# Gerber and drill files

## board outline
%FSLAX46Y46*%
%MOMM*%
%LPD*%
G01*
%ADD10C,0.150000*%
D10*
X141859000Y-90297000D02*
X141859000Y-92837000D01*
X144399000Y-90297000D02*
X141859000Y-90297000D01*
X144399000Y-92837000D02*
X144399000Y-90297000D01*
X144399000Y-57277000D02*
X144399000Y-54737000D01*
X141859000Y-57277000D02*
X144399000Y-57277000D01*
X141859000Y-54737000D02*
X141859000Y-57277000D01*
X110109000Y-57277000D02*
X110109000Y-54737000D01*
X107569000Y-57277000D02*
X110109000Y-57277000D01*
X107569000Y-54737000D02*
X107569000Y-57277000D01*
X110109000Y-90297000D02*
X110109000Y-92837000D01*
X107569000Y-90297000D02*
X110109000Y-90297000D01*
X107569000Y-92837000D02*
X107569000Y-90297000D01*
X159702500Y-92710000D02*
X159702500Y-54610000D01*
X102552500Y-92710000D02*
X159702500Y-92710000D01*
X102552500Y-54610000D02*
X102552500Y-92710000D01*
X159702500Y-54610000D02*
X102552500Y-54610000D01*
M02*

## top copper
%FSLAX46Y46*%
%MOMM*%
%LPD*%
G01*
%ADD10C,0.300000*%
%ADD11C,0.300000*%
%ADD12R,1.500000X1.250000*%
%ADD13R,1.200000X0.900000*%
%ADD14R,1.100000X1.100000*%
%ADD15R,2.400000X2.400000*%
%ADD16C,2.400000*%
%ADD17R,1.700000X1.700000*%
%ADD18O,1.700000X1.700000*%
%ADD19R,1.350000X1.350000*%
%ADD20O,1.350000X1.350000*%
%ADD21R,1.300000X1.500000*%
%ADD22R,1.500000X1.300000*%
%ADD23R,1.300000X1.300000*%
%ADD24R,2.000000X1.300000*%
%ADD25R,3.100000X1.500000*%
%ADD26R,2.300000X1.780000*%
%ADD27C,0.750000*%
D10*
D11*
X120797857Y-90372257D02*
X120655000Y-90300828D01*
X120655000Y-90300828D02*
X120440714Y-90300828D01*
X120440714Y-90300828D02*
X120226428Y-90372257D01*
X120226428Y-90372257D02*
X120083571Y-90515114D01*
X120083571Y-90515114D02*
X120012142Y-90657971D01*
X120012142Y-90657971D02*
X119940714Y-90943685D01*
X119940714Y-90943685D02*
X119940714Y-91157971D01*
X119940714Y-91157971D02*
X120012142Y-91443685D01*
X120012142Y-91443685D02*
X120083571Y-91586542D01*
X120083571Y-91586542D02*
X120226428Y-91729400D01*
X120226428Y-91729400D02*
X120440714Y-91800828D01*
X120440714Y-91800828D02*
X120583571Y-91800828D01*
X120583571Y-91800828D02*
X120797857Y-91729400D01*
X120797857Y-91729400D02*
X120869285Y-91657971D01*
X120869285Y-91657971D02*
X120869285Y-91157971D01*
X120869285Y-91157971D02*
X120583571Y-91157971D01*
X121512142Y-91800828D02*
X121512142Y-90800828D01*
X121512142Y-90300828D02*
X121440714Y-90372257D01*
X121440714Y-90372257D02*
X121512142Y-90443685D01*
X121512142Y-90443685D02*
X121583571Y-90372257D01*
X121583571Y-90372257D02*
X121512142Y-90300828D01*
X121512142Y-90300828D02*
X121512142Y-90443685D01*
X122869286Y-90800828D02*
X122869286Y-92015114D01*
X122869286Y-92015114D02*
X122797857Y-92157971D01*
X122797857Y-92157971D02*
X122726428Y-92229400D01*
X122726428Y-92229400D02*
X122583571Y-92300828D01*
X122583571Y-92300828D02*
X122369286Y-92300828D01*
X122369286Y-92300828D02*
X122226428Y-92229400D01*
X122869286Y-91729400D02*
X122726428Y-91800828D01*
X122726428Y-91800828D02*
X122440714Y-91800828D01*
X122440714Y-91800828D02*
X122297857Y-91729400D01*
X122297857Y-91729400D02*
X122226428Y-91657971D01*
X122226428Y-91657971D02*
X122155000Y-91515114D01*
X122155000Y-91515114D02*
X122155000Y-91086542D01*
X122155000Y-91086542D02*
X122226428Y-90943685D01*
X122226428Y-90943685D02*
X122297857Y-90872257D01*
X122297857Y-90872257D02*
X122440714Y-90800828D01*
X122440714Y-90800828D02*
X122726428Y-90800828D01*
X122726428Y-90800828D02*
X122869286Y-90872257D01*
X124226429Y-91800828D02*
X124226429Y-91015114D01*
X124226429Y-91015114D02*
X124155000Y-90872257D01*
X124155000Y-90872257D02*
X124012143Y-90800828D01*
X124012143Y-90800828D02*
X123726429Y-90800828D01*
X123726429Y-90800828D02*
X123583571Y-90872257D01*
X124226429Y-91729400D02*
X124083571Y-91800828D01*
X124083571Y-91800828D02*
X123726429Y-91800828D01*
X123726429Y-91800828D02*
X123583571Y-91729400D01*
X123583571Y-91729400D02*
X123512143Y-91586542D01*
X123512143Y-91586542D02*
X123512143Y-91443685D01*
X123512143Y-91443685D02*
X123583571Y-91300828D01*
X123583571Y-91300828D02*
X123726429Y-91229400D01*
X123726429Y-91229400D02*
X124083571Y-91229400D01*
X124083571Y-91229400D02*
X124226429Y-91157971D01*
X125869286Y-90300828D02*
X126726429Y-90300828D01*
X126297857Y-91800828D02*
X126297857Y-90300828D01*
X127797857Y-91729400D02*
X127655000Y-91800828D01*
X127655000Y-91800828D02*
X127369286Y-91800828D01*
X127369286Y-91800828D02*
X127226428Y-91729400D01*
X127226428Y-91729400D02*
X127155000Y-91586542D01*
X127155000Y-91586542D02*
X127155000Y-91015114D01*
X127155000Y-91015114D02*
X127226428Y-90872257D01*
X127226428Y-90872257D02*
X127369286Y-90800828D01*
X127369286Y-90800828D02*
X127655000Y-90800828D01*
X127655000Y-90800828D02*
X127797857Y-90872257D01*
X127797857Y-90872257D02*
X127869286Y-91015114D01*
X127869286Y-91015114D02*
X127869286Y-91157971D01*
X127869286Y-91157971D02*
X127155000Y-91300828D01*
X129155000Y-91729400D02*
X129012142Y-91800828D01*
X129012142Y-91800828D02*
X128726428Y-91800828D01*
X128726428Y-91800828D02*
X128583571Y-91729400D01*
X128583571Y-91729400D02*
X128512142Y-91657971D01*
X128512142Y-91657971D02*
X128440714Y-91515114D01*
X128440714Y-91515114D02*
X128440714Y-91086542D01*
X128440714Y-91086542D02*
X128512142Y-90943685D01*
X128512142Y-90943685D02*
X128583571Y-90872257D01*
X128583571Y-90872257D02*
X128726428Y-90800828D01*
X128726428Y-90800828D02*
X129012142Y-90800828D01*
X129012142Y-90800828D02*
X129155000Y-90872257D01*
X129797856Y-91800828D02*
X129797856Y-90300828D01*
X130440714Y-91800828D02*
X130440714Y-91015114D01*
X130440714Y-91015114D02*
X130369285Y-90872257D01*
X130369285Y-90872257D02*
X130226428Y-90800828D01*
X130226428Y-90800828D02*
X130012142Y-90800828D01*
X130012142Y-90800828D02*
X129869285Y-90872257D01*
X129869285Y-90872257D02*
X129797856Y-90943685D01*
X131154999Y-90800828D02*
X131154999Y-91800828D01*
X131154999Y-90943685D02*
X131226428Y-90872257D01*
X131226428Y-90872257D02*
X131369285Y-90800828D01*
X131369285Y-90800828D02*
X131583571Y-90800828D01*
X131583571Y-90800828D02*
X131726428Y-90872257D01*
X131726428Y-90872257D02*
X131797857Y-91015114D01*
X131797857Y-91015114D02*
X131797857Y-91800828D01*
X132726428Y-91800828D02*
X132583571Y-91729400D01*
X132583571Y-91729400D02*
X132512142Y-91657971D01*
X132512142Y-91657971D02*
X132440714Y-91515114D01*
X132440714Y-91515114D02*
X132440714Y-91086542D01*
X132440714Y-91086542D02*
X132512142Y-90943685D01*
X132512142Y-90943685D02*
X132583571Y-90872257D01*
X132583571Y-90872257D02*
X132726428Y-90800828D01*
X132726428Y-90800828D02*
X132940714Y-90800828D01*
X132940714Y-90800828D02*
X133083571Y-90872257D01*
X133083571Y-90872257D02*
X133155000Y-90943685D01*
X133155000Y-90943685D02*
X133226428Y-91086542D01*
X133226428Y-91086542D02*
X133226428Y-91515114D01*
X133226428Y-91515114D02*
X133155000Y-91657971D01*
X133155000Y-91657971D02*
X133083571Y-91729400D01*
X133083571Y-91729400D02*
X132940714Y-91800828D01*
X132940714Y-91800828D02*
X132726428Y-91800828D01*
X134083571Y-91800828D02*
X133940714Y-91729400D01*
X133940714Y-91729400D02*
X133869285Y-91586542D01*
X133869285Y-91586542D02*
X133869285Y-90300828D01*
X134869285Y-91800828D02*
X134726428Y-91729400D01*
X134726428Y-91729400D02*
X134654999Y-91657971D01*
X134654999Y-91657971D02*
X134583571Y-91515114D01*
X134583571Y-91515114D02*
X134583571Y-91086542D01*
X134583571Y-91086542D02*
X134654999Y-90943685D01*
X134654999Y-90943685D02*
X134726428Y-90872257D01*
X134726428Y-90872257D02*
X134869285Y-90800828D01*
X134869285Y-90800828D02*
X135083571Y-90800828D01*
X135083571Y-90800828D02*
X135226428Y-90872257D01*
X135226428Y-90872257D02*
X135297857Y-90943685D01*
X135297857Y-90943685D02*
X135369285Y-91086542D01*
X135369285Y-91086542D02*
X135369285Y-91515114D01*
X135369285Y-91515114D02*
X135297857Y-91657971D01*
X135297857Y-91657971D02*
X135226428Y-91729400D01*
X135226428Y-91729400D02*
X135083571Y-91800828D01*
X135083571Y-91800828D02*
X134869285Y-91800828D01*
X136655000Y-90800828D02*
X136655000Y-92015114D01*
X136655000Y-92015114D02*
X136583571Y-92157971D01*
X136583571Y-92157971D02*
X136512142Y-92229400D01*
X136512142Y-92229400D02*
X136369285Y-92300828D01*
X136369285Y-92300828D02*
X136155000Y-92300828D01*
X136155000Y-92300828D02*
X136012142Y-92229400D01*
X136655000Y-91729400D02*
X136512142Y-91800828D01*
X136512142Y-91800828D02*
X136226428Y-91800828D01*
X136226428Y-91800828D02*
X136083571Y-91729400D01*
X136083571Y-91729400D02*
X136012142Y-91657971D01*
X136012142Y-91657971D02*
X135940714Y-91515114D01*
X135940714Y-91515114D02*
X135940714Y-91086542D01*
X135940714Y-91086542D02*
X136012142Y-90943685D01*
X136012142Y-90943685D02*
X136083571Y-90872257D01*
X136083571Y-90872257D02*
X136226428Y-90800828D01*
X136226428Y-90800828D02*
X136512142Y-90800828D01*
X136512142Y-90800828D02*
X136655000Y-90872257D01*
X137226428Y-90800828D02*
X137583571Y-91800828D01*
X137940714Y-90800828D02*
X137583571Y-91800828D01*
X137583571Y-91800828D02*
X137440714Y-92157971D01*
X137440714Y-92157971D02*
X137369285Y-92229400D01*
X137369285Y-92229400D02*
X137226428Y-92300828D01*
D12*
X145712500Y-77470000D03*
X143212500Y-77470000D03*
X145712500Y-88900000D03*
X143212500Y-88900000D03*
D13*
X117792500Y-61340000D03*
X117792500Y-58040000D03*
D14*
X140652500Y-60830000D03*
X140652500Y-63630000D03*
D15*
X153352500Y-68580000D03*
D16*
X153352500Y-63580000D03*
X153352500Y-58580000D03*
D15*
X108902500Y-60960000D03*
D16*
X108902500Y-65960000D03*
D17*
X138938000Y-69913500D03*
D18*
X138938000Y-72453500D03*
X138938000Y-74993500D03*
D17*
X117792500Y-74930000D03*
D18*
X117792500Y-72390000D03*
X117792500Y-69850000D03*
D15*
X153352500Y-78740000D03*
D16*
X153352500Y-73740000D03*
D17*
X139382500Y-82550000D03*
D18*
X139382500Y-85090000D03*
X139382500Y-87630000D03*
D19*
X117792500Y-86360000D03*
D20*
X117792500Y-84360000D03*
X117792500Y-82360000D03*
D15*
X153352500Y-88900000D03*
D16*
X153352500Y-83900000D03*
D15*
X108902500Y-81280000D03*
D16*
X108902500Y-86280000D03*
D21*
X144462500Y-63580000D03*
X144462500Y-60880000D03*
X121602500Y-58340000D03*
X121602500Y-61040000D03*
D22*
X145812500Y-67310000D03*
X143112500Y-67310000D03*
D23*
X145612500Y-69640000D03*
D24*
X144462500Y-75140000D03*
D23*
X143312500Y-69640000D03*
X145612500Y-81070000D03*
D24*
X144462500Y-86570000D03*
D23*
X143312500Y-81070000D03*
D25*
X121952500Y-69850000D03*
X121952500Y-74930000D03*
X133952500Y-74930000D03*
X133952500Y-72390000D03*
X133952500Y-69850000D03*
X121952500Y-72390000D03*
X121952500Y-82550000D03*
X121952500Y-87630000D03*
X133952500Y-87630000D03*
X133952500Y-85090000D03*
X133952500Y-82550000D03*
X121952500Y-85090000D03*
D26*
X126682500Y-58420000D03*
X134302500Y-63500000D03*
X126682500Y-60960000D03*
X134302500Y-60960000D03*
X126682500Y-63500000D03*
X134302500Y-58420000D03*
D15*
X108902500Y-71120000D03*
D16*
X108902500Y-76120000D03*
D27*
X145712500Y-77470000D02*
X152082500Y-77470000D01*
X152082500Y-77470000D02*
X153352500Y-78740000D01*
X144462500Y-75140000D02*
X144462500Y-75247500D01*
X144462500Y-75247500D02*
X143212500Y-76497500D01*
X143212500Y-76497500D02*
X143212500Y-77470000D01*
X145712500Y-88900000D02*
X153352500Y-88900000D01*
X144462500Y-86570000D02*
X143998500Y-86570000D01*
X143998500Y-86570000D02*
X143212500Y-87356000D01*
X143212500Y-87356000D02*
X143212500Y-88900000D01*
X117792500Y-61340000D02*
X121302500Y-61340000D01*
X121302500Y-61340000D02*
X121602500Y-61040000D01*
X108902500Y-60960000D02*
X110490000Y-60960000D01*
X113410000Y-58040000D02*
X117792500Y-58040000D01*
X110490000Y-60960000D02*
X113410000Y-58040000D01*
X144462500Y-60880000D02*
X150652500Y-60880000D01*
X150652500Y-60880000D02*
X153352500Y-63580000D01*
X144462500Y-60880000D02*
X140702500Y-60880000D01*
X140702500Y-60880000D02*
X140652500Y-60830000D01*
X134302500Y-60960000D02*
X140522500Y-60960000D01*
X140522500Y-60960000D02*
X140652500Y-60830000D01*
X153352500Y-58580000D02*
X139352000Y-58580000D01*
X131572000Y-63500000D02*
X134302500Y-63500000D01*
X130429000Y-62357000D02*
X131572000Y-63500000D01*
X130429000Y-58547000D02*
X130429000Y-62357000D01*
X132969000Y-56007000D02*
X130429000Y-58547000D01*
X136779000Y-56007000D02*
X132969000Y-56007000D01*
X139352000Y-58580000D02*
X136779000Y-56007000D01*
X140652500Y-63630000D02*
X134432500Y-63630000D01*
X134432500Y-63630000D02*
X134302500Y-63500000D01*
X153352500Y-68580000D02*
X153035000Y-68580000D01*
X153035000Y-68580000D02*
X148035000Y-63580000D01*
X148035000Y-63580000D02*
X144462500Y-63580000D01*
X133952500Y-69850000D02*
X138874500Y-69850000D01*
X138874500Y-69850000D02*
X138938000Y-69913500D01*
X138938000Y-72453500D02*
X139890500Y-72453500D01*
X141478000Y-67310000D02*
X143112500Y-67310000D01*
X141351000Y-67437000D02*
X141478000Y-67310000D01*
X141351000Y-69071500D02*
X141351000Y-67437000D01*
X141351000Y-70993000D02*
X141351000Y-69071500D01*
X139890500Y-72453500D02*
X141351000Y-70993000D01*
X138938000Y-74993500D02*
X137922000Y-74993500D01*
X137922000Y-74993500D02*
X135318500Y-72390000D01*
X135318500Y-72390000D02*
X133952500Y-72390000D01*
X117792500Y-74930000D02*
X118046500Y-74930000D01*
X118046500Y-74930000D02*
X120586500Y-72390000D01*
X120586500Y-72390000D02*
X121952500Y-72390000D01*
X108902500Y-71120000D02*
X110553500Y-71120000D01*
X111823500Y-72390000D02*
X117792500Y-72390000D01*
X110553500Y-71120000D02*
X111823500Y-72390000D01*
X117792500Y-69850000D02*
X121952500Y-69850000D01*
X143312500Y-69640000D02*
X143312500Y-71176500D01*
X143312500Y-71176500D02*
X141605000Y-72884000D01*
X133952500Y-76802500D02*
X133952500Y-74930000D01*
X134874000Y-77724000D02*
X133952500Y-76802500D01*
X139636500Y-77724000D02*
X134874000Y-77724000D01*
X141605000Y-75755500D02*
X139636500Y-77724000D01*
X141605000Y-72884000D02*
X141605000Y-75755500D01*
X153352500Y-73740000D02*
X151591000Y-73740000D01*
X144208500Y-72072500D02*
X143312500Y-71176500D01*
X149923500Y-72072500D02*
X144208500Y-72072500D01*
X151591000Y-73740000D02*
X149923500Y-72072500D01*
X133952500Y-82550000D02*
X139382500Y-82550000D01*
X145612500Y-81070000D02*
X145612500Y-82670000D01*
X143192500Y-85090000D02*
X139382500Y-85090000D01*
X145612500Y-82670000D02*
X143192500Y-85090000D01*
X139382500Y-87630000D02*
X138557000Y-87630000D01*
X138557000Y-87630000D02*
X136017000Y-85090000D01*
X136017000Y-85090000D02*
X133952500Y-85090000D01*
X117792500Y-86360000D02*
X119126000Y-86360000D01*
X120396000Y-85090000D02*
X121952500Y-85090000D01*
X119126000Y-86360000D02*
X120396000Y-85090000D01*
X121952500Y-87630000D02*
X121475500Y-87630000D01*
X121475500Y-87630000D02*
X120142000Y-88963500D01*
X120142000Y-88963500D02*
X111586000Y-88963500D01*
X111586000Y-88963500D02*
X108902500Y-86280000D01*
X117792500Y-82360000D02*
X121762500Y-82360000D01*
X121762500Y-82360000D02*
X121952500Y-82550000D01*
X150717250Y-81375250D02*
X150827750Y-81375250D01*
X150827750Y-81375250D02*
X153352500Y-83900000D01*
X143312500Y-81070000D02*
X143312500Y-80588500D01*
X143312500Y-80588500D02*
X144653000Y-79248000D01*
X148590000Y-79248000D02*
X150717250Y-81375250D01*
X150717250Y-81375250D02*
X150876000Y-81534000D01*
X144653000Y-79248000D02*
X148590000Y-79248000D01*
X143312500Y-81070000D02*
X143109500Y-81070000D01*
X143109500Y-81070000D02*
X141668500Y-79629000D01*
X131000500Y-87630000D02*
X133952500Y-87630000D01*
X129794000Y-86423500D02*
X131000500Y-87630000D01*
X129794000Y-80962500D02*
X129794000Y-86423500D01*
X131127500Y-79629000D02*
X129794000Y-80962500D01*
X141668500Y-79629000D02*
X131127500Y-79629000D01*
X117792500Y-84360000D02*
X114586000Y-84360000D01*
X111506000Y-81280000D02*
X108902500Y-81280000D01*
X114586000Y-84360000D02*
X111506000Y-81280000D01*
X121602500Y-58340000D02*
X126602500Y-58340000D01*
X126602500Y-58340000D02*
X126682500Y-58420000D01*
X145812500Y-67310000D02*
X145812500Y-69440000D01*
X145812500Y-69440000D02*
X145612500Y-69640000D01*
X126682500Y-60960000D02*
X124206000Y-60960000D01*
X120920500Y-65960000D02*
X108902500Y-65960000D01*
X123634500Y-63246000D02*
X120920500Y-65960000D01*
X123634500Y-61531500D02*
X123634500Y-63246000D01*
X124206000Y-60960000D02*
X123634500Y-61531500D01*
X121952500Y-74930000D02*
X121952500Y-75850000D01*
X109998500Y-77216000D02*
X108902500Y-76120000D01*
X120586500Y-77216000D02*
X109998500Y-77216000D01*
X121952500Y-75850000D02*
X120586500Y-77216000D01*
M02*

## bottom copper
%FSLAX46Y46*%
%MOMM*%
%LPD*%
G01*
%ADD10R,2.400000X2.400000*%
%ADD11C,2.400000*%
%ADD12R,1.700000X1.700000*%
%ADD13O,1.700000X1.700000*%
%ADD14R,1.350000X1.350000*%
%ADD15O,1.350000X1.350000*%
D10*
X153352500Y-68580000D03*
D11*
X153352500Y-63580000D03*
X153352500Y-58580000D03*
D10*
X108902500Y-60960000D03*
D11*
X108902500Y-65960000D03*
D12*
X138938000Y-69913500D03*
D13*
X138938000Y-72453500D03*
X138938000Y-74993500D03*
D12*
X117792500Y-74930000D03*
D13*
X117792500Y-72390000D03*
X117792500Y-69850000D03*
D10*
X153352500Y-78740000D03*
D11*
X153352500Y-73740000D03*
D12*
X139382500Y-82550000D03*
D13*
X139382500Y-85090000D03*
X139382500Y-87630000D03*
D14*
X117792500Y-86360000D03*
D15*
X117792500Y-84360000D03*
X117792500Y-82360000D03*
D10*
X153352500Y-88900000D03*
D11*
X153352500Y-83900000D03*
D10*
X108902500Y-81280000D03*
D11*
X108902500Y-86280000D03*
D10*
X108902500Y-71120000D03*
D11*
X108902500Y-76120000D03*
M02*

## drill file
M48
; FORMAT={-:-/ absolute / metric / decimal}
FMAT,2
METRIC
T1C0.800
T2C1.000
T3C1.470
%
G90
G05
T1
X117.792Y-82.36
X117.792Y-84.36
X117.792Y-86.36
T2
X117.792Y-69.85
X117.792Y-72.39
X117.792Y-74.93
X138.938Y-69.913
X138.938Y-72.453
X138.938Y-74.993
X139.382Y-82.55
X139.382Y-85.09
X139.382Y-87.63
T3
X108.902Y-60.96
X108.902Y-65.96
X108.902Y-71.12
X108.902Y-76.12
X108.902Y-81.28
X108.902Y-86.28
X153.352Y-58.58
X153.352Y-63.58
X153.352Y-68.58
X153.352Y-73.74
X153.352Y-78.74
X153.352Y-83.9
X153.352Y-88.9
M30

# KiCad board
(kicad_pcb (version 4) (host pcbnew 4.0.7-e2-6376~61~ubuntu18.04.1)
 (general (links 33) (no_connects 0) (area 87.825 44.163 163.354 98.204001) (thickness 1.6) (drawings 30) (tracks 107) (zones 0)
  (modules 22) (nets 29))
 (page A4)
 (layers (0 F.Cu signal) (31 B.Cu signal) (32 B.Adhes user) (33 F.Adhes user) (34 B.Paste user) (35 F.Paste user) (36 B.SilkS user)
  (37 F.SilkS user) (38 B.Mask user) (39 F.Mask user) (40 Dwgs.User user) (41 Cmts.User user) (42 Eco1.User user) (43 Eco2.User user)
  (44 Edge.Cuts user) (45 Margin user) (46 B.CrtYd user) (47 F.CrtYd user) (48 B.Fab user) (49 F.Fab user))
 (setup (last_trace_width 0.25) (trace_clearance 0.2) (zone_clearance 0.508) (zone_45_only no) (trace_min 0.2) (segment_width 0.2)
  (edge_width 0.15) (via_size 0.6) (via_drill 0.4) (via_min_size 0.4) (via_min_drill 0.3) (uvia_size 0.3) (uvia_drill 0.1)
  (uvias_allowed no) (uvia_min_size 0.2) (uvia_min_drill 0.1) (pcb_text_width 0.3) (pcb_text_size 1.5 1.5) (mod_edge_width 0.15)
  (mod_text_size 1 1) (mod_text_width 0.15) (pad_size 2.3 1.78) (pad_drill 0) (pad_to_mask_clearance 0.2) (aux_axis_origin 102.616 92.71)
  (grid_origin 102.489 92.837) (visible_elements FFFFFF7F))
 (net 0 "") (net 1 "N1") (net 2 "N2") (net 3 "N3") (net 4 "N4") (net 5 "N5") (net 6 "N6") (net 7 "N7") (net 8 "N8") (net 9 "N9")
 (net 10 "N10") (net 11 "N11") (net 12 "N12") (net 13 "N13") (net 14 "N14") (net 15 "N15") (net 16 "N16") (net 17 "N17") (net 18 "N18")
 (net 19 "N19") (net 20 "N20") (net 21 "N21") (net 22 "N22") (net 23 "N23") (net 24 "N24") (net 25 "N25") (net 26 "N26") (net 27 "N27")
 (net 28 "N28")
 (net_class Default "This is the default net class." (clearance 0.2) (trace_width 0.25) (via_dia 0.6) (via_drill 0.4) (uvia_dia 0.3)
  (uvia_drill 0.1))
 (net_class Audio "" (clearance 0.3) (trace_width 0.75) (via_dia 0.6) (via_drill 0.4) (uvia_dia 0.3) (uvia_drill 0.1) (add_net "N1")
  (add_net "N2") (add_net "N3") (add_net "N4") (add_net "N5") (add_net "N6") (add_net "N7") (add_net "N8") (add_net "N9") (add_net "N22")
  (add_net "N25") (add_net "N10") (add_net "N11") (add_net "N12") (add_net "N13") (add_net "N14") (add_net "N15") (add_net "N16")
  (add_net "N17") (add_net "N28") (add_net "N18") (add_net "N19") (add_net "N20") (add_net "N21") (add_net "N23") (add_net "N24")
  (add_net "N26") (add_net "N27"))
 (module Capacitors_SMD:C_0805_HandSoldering (layer F.Cu) (at 144.4625 77.47 180)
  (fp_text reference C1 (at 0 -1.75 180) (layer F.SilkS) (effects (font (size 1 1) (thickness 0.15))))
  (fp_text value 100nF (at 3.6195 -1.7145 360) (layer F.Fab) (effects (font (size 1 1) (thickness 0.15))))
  (pad 1 smd rect (at -1.25 0 180) (size 1.5 1.25) (layers F.Cu F.Paste F.Mask) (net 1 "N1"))
  (pad 2 smd rect (at 1.25 0 180) (size 1.5 1.25) (layers F.Cu F.Paste F.Mask) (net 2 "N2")))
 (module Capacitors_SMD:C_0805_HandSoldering (layer F.Cu) (at 144.4625 88.9 180)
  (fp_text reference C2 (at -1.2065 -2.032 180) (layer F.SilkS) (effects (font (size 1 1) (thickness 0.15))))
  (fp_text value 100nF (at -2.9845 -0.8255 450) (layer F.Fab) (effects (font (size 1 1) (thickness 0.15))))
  (pad 1 smd rect (at -1.25 0 180) (size 1.5 1.25) (layers F.Cu F.Paste F.Mask) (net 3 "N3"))
  (pad 2 smd rect (at 1.25 0 180) (size 1.5 1.25) (layers F.Cu F.Paste F.Mask) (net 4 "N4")))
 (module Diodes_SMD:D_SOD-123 (layer F.Cu) (at 117.7925 59.69 90)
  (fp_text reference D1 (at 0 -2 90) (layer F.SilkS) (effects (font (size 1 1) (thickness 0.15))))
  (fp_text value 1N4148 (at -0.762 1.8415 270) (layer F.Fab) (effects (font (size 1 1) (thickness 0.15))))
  (pad 1 smd rect (at -1.65 0 90) (size 0.9 1.2) (layers F.Cu F.Paste F.Mask) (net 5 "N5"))
  (pad 2 smd rect (at 1.65 0 90) (size 0.9 1.2) (layers F.Cu F.Paste F.Mask) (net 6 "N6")))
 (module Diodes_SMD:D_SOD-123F (layer F.Cu) (at 140.6525 62.23 270)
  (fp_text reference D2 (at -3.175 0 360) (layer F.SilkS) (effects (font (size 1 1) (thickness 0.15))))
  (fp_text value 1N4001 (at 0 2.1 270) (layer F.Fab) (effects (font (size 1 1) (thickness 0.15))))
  (pad 1 smd rect (at -1.4 0 270) (size 1.1 1.1) (layers F.Cu F.Paste F.Mask) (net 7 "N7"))
  (pad 2 smd rect (at 1.4 0 270) (size 1.1 1.1) (layers F.Cu F.Paste F.Mask) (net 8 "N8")))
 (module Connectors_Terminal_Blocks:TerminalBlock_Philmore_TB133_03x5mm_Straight (layer F.Cu) (at 153.3525 68.58 90)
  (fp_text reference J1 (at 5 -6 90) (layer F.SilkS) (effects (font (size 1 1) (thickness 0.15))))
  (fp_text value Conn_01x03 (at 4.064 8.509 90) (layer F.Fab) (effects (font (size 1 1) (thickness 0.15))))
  (pad 1 thru_hole rect (at 0 0 90) (size 2.4 2.4) (drill 1.47) (layers *.Cu *.Mask) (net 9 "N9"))
  (pad 2 thru_hole circle (at 5 0 90) (size 2.4 2.4) (drill 1.47) (layers *.Cu *.Mask) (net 7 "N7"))
  (pad 3 thru_hole circle (at 10 0 90) (size 2.4 2.4) (drill 1.47) (layers *.Cu *.Mask) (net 8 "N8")))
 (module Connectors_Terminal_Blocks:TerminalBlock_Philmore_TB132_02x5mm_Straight (layer F.Cu) (at 108.9025 60.96 270)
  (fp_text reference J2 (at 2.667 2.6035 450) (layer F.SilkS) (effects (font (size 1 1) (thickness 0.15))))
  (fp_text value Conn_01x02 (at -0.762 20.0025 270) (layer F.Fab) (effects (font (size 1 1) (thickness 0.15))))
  (pad 1 thru_hole rect (at 0 0 270) (size 2.4 2.4) (drill 1.47) (layers *.Cu *.Mask) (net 6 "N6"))
  (pad 2 thru_hole circle (at 5 0 270) (size 2.4 2.4) (drill 1.47) (layers *.Cu *.Mask) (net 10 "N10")))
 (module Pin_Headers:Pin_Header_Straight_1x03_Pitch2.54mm (layer F.Cu) (at 138.938 69.9135)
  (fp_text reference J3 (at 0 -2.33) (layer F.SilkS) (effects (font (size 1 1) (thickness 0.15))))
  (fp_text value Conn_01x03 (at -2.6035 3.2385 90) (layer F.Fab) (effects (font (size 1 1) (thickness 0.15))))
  (pad 1 thru_hole rect (at 0 0) (size 1.7 1.7) (drill 1) (layers *.Cu *.Mask) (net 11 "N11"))
  (pad 2 thru_hole oval (at 0 2.54) (size 1.7 1.7) (drill 1) (layers *.Cu *.Mask) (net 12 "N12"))
  (pad 3 thru_hole oval (at 0 5.08) (size 1.7 1.7) (drill 1) (layers *.Cu *.Mask) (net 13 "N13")))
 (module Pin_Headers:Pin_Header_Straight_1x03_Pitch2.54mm (layer F.Cu) (at 117.7925 74.93 180)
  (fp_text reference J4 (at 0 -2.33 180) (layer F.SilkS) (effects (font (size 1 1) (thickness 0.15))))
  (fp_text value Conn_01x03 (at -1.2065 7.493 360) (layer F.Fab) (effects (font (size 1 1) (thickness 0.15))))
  (pad 1 thru_hole rect (at 0 0 180) (size 1.7 1.7) (drill 1) (layers *.Cu *.Mask) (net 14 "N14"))
  (pad 2 thru_hole oval (at 0 2.54 180) (size 1.7 1.7) (drill 1) (layers *.Cu *.Mask) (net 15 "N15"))
  (pad 3 thru_hole oval (at 0 5.08 180) (size 1.7 1.7) (drill 1) (layers *.Cu *.Mask) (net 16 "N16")))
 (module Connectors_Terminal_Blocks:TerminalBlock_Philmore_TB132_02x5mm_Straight (layer F.Cu) (at 153.3525 78.74 90)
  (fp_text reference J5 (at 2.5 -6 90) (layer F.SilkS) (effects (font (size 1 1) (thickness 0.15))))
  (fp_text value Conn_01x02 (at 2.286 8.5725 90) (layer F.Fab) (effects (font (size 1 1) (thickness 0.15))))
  (pad 1 thru_hole rect (at 0 0 90) (size 2.4 2.4) (drill 1.47) (layers *.Cu *.Mask) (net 1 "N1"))
  (pad 2 thru_hole circle (at 5 0 90) (size 2.4 2.4) (drill 1.47) (layers *.Cu *.Mask) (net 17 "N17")))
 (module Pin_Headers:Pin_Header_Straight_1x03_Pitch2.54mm (layer F.Cu) (at 139.3825 82.55)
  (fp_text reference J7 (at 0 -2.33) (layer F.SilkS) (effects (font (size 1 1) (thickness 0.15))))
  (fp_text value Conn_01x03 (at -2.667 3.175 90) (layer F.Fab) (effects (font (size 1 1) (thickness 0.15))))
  (pad 1 thru_hole rect (at 0 0) (size 1.7 1.7) (drill 1) (layers *.Cu *.Mask) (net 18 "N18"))
  (pad 2 thru_hole oval (at 0 2.54) (size 1.7 1.7) (drill 1) (layers *.Cu *.Mask) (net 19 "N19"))
  (pad 3 thru_hole oval (at 0 5.08) (size 1.7 1.7) (drill 1) (layers *.Cu *.Mask) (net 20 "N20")))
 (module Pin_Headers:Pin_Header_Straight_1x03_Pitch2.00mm (layer F.Cu) (at 117.7925 86.36 180)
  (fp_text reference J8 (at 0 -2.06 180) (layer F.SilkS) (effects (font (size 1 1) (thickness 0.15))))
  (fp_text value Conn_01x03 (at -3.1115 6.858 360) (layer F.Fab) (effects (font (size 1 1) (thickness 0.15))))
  (pad 1 thru_hole rect (at 0 0 180) (size 1.35 1.35) (drill 0.8) (layers *.Cu *.Mask) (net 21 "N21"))
  (pad 2 thru_hole oval (at 0 2 180) (size 1.35 1.35) (drill 0.8) (layers *.Cu *.Mask) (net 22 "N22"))
  (pad 3 thru_hole oval (at 0 4 180) (size 1.35 1.35) (drill 0.8) (layers *.Cu *.Mask) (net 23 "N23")))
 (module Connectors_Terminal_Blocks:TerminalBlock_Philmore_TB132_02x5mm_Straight (layer F.Cu) (at 153.3525 88.9 90)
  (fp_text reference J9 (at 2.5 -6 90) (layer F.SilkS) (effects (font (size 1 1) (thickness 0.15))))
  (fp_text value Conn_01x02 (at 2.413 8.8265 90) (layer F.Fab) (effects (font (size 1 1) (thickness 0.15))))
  (pad 1 thru_hole rect (at 0 0 90) (size 2.4 2.4) (drill 1.47) (layers *.Cu *.Mask) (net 3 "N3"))
  (pad 2 thru_hole circle (at 5 0 90) (size 2.4 2.4) (drill 1.47) (layers *.Cu *.Mask) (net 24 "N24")))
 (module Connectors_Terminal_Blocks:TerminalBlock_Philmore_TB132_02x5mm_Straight (layer F.Cu) (at 108.9025 81.28 270)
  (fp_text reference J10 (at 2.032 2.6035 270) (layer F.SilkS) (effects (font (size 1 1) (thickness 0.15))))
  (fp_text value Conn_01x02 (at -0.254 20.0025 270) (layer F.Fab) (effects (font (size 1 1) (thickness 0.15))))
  (pad 1 thru_hole rect (at 0 0 270) (size 2.4 2.4) (drill 1.47) (layers *.Cu *.Mask) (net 22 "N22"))
  (pad 2 thru_hole circle (at 5 0 270) (size 2.4 2.4) (drill 1.47) (layers *.Cu *.Mask) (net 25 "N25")))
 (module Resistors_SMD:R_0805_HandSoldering (layer F.Cu) (at 144.4625 62.23 90)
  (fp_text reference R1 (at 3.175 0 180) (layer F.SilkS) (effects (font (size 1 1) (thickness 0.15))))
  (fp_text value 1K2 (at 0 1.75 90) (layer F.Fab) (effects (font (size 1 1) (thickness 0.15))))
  (pad 1 smd rect (at -1.35 0 90) (size 1.5 1.3) (layers F.Cu F.Paste F.Mask) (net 9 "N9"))
  (pad 2 smd rect (at 1.35 0 90) (size 1.5 1.3) (layers F.Cu F.Paste F.Mask) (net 7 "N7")))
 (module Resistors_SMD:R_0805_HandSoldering (layer F.Cu) (at 121.6025 59.69 270)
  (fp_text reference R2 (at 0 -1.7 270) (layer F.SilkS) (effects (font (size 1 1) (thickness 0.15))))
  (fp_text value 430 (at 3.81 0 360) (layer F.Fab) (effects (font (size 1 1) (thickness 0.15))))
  (pad 1 smd rect (at -1.35 0 270) (size 1.5 1.3) (layers F.Cu F.Paste F.Mask) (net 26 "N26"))
  (pad 2 smd rect (at 1.35 0 270) (size 1.5 1.3) (layers F.Cu F.Paste F.Mask) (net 5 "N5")))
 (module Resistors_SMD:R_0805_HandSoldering (layer F.Cu) (at 144.4625 67.31 180)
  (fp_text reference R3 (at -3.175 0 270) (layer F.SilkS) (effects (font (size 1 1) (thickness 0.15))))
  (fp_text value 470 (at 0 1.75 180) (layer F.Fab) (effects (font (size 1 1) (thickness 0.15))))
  (pad 1 smd rect (at -1.35 0 180) (size 1.5 1.3) (layers F.Cu F.Paste F.Mask) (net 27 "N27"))
  (pad 2 smd rect (at 1.35 0 180) (size 1.5 1.3) (layers F.Cu F.Paste F.Mask) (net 12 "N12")))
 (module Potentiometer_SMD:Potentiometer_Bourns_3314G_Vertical (layer F.Cu) (at 144.4625 72.39)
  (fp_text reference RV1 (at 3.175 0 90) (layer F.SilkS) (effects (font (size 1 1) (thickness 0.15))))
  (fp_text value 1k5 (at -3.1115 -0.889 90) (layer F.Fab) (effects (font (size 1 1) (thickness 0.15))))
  (pad 1 smd rect (at 1.15 -2.75) (size 1.3 1.3) (layers F.Cu F.Paste F.Mask) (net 27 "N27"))
  (pad 2 smd rect (at 0 2.75) (size 2 1.3) (layers F.Cu F.Paste F.Mask) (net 2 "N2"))
  (pad 3 smd rect (at -1.15 -2.75) (size 1.3 1.3) (layers F.Cu F.Paste F.Mask) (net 17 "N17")))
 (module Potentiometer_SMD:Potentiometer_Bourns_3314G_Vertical (layer F.Cu) (at 144.4625 83.82)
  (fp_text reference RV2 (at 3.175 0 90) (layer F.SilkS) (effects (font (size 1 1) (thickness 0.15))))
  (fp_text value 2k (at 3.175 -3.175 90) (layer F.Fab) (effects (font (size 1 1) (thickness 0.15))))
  (pad 1 smd rect (at 1.15 -2.75) (size 1.3 1.3) (layers F.Cu F.Paste F.Mask) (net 19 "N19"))
  (pad 2 smd rect (at 0 2.75) (size 2 1.3) (layers F.Cu F.Paste F.Mask) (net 4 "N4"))
  (pad 3 smd rect (at -1.15 -2.75) (size 1.3 1.3) (layers F.Cu F.Paste F.Mask) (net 24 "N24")))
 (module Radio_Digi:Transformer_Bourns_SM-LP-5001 (layer F.Cu) (at 127.9525 72.39)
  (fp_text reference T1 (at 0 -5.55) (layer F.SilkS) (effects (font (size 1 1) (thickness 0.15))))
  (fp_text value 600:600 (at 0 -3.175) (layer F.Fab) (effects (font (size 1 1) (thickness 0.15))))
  (pad 1 smd rect (at -6 -2.54) (size 3.1 1.5) (layers F.Cu F.Paste F.Mask) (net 16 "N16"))
  (pad 3 smd rect (at -6 2.54) (size 3.1 1.5) (layers F.Cu F.Paste F.Mask) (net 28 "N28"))
  (pad 4 smd rect (at 6 2.54) (size 3.1 1.5) (layers F.Cu F.Paste F.Mask) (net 17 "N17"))
  (pad 5 smd rect (at 6 0) (size 3.1 1.5) (layers F.Cu F.Paste F.Mask) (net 13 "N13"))
  (pad 6 smd rect (at 6 -2.54) (size 3.1 1.5) (layers F.Cu F.Paste F.Mask) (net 11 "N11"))
  (pad 2 smd rect (at -6 0) (size 3.1 1.5) (layers F.Cu F.Paste F.Mask) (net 14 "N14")))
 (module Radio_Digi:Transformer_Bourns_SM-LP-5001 (layer F.Cu) (at 127.9525 85.09)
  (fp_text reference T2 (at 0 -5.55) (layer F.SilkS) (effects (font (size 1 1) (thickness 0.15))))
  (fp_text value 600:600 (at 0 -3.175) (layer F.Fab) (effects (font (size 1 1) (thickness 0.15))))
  (pad 1 smd rect (at -6 -2.54) (size 3.1 1.5) (layers F.Cu F.Paste F.Mask) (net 23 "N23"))
  (pad 3 smd rect (at -6 2.54) (size 3.1 1.5) (layers F.Cu F.Paste F.Mask) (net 25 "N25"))
  (pad 4 smd rect (at 6 2.54) (size 3.1 1.5) (layers F.Cu F.Paste F.Mask) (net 24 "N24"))
  (pad 5 smd rect (at 6 0) (size 3.1 1.5) (layers F.Cu F.Paste F.Mask) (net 20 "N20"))
  (pad 6 smd rect (at 6 -2.54) (size 3.1 1.5) (layers F.Cu F.Paste F.Mask) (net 18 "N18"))
  (pad 2 smd rect (at -6 0) (size 3.1 1.5) (layers F.Cu F.Paste F.Mask) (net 21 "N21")))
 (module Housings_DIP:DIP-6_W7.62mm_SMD (layer F.Cu) (at 130.4925 60.96)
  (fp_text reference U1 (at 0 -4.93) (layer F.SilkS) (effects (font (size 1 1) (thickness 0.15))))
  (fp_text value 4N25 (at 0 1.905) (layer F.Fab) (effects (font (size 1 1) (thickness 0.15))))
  (pad 1 smd rect (at -3.81 -2.54) (size 2.3 1.78) (layers F.Cu F.Paste F.Mask) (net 26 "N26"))
  (pad 4 smd rect (at 3.81 2.54) (size 2.3 1.78) (layers F.Cu F.Paste F.Mask) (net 8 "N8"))
  (pad 2 smd rect (at -3.81 0) (size 2.3 1.78) (layers F.Cu F.Paste F.Mask) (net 10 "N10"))
  (pad 5 smd rect (at 3.81 0) (size 2.3 1.78) (layers F.Cu F.Paste F.Mask) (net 7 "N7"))
  (pad 3 smd rect (at -3.81 2.54) (size 2.3 1.78) (layers F.Cu F.Paste F.Mask))
  (pad 6 smd rect (at 3.81 -2.54) (size 2.3 1.78) (layers F.Cu F.Paste F.Mask)))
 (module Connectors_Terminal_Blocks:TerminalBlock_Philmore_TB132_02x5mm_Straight (layer F.Cu) (at 108.9025 71.12 270)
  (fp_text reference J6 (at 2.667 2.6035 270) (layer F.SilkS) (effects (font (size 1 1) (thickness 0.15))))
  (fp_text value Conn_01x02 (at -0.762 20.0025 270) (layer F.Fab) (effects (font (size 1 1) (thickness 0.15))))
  (pad 1 thru_hole rect (at 0 0 270) (size 2.4 2.4) (drill 1.47) (layers *.Cu *.Mask) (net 15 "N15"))
  (pad 2 thru_hole circle (at 5 0 270) (size 2.4 2.4) (drill 1.47) (layers *.Cu *.Mask) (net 28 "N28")))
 (gr_line (start 141.859 90.297) (end 141.859 92.837) (angle 90) (layer Edge.Cuts) (width 0.15))
 (gr_line (start 144.399 90.297) (end 141.859 90.297) (angle 90) (layer Edge.Cuts) (width 0.15))
 (gr_line (start 144.399 92.837) (end 144.399 90.297) (angle 90) (layer Edge.Cuts) (width 0.15))
 (gr_line (start 144.399 57.277) (end 144.399 54.737) (angle 90) (layer Edge.Cuts) (width 0.15))
 (gr_line (start 141.859 57.277) (end 144.399 57.277) (angle 90) (layer Edge.Cuts) (width 0.15))
 (gr_line (start 141.859 54.737) (end 141.859 57.277) (angle 90) (layer Edge.Cuts) (width 0.15))
 (gr_line (start 110.109 57.277) (end 110.109 54.737) (angle 90) (layer Edge.Cuts) (width 0.15))
 (gr_line (start 107.569 57.277) (end 110.109 57.277) (angle 90) (layer Edge.Cuts) (width 0.15))
 (gr_line (start 107.569 54.737) (end 107.569 57.277) (angle 90) (layer Edge.Cuts) (width 0.15))
 (gr_line (start 110.109 90.297) (end 110.109 92.837) (angle 90) (layer Edge.Cuts) (width 0.15))
 (gr_line (start 107.569 90.297) (end 110.109 90.297) (angle 90) (layer Edge.Cuts) (width 0.15))
 (gr_line (start 107.569 92.837) (end 107.569 90.297) (angle 90) (layer Edge.Cuts) (width 0.15))
 (gr_line (start 159.7025 92.71) (end 159.7025 54.61) (angle 90) (layer Edge.Cuts) (width 0.15))
 (gr_line (start 102.5525 92.71) (end 159.7025 92.71) (angle 90) (layer Edge.Cuts) (width 0.15))
 (gr_line (start 102.5525 54.61) (end 102.5525 92.71) (angle 90) (layer Edge.Cuts) (width 0.15))
 (gr_line (start 159.7025 54.61) (end 102.5525 54.61) (angle 90) (layer Edge.Cuts) (width 0.15))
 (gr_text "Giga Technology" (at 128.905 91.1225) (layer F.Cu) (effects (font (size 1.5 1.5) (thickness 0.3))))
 (segment (start 145.7125 77.47) (end 152.0825 77.47) (width 0.75) (layer F.Cu) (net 1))
 (segment (start 152.0825 77.47) (end 153.3525 78.74) (width 0.75) (layer F.Cu) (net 1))
 (segment (start 144.4625 75.14) (end 144.4625 75.2475) (width 0.75) (layer F.Cu) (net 2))
 (segment (start 144.4625 75.2475) (end 143.2125 76.4975) (width 0.75) (layer F.Cu) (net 2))
 (segment (start 143.2125 76.4975) (end 143.2125 77.47) (width 0.75) (layer F.Cu) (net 2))
 (segment (start 145.7125 88.9) (end 153.3525 88.9) (width 0.75) (layer F.Cu) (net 3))
 (segment (start 144.4625 86.57) (end 143.9985 86.57) (width 0.75) (layer F.Cu) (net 4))
 (segment (start 143.9985 86.57) (end 143.2125 87.356) (width 0.75) (layer F.Cu) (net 4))
 (segment (start 143.2125 87.356) (end 143.2125 88.9) (width 0.75) (layer F.Cu) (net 4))
 (segment (start 117.7925 61.34) (end 121.3025 61.34) (width 0.75) (layer F.Cu) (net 5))
 (segment (start 121.3025 61.34) (end 121.6025 61.04) (width 0.75) (layer F.Cu) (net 5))
 (segment (start 108.9025 60.96) (end 110.49 60.96) (width 0.75) (layer F.Cu) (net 6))
 (segment (start 113.41 58.04) (end 117.7925 58.04) (width 0.75) (layer F.Cu) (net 6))
 (segment (start 110.49 60.96) (end 113.41 58.04) (width 0.75) (layer F.Cu) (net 6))
 (segment (start 144.4625 60.88) (end 150.6525 60.88) (width 0.75) (layer F.Cu) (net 7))
 (segment (start 150.6525 60.88) (end 153.3525 63.58) (width 0.75) (layer F.Cu) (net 7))
 (segment (start 144.4625 60.88) (end 140.7025 60.88) (width 0.75) (layer F.Cu) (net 7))
 (segment (start 140.7025 60.88) (end 140.6525 60.83) (width 0.75) (layer F.Cu) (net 7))
 (segment (start 134.3025 60.96) (end 140.5225 60.96) (width 0.75) (layer F.Cu) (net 7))
 (segment (start 140.5225 60.96) (end 140.6525 60.83) (width 0.75) (layer F.Cu) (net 7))
 (segment (start 153.3525 58.58) (end 139.352 58.58) (width 0.75) (layer F.Cu) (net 8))
 (segment (start 131.572 63.5) (end 134.3025 63.5) (width 0.75) (layer F.Cu) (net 8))
 (segment (start 130.429 62.357) (end 131.572 63.5) (width 0.75) (layer F.Cu) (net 8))
 (segment (start 130.429 58.547) (end 130.429 62.357) (width 0.75) (layer F.Cu) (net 8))
 (segment (start 132.969 56.007) (end 130.429 58.547) (width 0.75) (layer F.Cu) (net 8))
 (segment (start 136.779 56.007) (end 132.969 56.007) (width 0.75) (layer F.Cu) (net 8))
 (segment (start 139.352 58.58) (end 136.779 56.007) (width 0.75) (layer F.Cu) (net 8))
 (segment (start 140.6525 63.63) (end 134.4325 63.63) (width 0.75) (layer F.Cu) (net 8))
 (segment (start 134.4325 63.63) (end 134.3025 63.5) (width 0.75) (layer F.Cu) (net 8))
 (segment (start 153.3525 68.58) (end 153.035 68.58) (width 0.75) (layer F.Cu) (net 9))
 (segment (start 153.035 68.58) (end 148.035 63.58) (width 0.75) (layer F.Cu) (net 9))
 (segment (start 148.035 63.58) (end 144.4625 63.58) (width 0.75) (layer F.Cu) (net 9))
 (segment (start 133.9525 69.85) (end 138.8745 69.85) (width 0.75) (layer F.Cu) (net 11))
 (segment (start 138.8745 69.85) (end 138.938 69.9135) (width 0.75) (layer F.Cu) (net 11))
 (segment (start 138.938 72.4535) (end 139.8905 72.4535) (width 0.75) (layer F.Cu) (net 12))
 (segment (start 141.478 67.31) (end 143.1125 67.31) (width 0.75) (layer F.Cu) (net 12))
 (segment (start 141.351 67.437) (end 141.478 67.31) (width 0.75) (layer F.Cu) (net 12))
 (segment (start 141.351 69.0715) (end 141.351 67.437) (width 0.75) (layer F.Cu) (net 12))
 (segment (start 141.351 70.993) (end 141.351 69.0715) (width 0.75) (layer F.Cu) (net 12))
 (segment (start 139.8905 72.4535) (end 141.351 70.993) (width 0.75) (layer F.Cu) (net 12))
 (segment (start 138.938 74.9935) (end 137.922 74.9935) (width 0.75) (layer F.Cu) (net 13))
 (segment (start 137.922 74.9935) (end 135.3185 72.39) (width 0.75) (layer F.Cu) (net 13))
 (segment (start 135.3185 72.39) (end 133.9525 72.39) (width 0.75) (layer F.Cu) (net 13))
 (segment (start 117.7925 74.93) (end 118.0465 74.93) (width 0.75) (layer F.Cu) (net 14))
 (segment (start 118.0465 74.93) (end 120.5865 72.39) (width 0.75) (layer F.Cu) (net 14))
 (segment (start 120.5865 72.39) (end 121.9525 72.39) (width 0.75) (layer F.Cu) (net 14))
 (segment (start 108.9025 71.12) (end 110.5535 71.12) (width 0.75) (layer F.Cu) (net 15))
 (segment (start 111.8235 72.39) (end 117.7925 72.39) (width 0.75) (layer F.Cu) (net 15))
 (segment (start 110.5535 71.12) (end 111.8235 72.39) (width 0.75) (layer F.Cu) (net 15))
 (segment (start 117.7925 69.85) (end 121.9525 69.85) (width 0.75) (layer F.Cu) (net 16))
 (segment (start 143.3125 69.64) (end 143.3125 71.1765) (width 0.75) (layer F.Cu) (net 17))
 (segment (start 143.3125 71.1765) (end 141.605 72.884) (width 0.75) (layer F.Cu) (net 17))
 (segment (start 133.9525 76.8025) (end 133.9525 74.93) (width 0.75) (layer F.Cu) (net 17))
 (segment (start 134.874 77.724) (end 133.9525 76.8025) (width 0.75) (layer F.Cu) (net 17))
 (segment (start 139.6365 77.724) (end 134.874 77.724) (width 0.75) (layer F.Cu) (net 17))
 (segment (start 141.605 75.7555) (end 139.6365 77.724) (width 0.75) (layer F.Cu) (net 17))
 (segment (start 141.605 72.884) (end 141.605 75.7555) (width 0.75) (layer F.Cu) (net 17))
 (segment (start 153.3525 73.74) (end 151.591 73.74) (width 0.75) (layer F.Cu) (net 17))
 (segment (start 144.2085 72.0725) (end 143.3125 71.1765) (width 0.75) (layer F.Cu) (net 17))
 (segment (start 149.9235 72.0725) (end 144.2085 72.0725) (width 0.75) (layer F.Cu) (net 17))
 (segment (start 151.591 73.74) (end 149.9235 72.0725) (width 0.75) (layer F.Cu) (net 17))
 (segment (start 133.9525 82.55) (end 139.3825 82.55) (width 0.75) (layer F.Cu) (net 18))
 (segment (start 145.6125 81.07) (end 145.6125 82.67) (width 0.75) (layer F.Cu) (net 19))
 (segment (start 143.1925 85.09) (end 139.3825 85.09) (width 0.75) (layer F.Cu) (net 19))
 (segment (start 145.6125 82.67) (end 143.1925 85.09) (width 0.75) (layer F.Cu) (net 19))
 (segment (start 139.3825 87.63) (end 138.557 87.63) (width 0.75) (layer F.Cu) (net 20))
 (segment (start 138.557 87.63) (end 136.017 85.09) (width 0.75) (layer F.Cu) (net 20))
 (segment (start 136.017 85.09) (end 133.9525 85.09) (width 0.75) (layer F.Cu) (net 20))
 (segment (start 117.7925 86.36) (end 119.126 86.36) (width 0.75) (layer F.Cu) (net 21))
 (segment (start 120.396 85.09) (end 121.9525 85.09) (width 0.75) (layer F.Cu) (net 21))
 (segment (start 119.126 86.36) (end 120.396 85.09) (width 0.75) (layer F.Cu) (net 21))
 (segment (start 121.9525 87.63) (end 121.4755 87.63) (width 0.75) (layer F.Cu) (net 25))
 (segment (start 121.4755 87.63) (end 120.142 88.9635) (width 0.75) (layer F.Cu) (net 25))
 (segment (start 120.142 88.9635) (end 111.586 88.9635) (width 0.75) (layer F.Cu) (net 25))
 (segment (start 111.586 88.9635) (end 108.9025 86.28) (width 0.75) (layer F.Cu) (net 25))
 (segment (start 117.7925 82.36) (end 121.7625 82.36) (width 0.75) (layer F.Cu) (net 23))
 (segment (start 121.7625 82.36) (end 121.9525 82.55) (width 0.75) (layer F.Cu) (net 23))
 (segment (start 150.71725 81.37525) (end 150.82775 81.37525) (width 0.75) (layer F.Cu) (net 24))
 (segment (start 150.82775 81.37525) (end 153.3525 83.9) (width 0.75) (layer F.Cu) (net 24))
 (segment (start 143.3125 81.07) (end 143.3125 80.5885) (width 0.75) (layer F.Cu) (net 24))
 (segment (start 143.3125 80.5885) (end 144.653 79.248) (width 0.75) (layer F.Cu) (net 24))
 (segment (start 148.59 79.248) (end 150.71725 81.37525) (width 0.75) (layer F.Cu) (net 24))
 (segment (start 150.71725 81.37525) (end 150.876 81.534) (width 0.75) (layer F.Cu) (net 24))
 (segment (start 144.653 79.248) (end 148.59 79.248) (width 0.75) (layer F.Cu) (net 24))
 (segment (start 143.3125 81.07) (end 143.1095 81.07) (width 0.75) (layer F.Cu) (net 24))
 (segment (start 143.1095 81.07) (end 141.6685 79.629) (width 0.75) (layer F.Cu) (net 24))
 (segment (start 131.0005 87.63) (end 133.9525 87.63) (width 0.75) (layer F.Cu) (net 24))
 (segment (start 129.794 86.4235) (end 131.0005 87.63) (width 0.75) (layer F.Cu) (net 24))
 (segment (start 129.794 80.9625) (end 129.794 86.4235) (width 0.75) (layer F.Cu) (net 24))
 (segment (start 131.1275 79.629) (end 129.794 80.9625) (width 0.75) (layer F.Cu) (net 24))
 (segment (start 141.6685 79.629) (end 131.1275 79.629) (width 0.75) (layer F.Cu) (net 24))
 (segment (start 117.7925 84.36) (end 114.586 84.36) (width 0.75) (layer F.Cu) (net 22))
 (segment (start 111.506 81.28) (end 108.9025 81.28) (width 0.75) (layer F.Cu) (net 22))
 (segment (start 114.586 84.36) (end 111.506 81.28) (width 0.75) (layer F.Cu) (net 22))
 (segment (start 121.6025 58.34) (end 126.6025 58.34) (width 0.75) (layer F.Cu) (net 26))
 (segment (start 126.6025 58.34) (end 126.6825 58.42) (width 0.75) (layer F.Cu) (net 26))
 (segment (start 145.8125 67.31) (end 145.8125 69.44) (width 0.75) (layer F.Cu) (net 27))
 (segment (start 145.8125 69.44) (end 145.6125 69.64) (width 0.75) (layer F.Cu) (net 27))
 (segment (start 126.6825 60.96) (end 124.206 60.96) (width 0.75) (layer F.Cu) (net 10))
 (segment (start 120.9205 65.96) (end 108.9025 65.96) (width 0.75) (layer F.Cu) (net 10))
 (segment (start 123.6345 63.246) (end 120.9205 65.96) (width 0.75) (layer F.Cu) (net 10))
 (segment (start 123.6345 61.5315) (end 123.6345 63.246) (width 0.75) (layer F.Cu) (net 10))
 (segment (start 124.206 60.96) (end 123.6345 61.5315) (width 0.75) (layer F.Cu) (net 10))
 (segment (start 121.9525 74.93) (end 121.9525 75.85) (width 0.75) (layer F.Cu) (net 28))
 (segment (start 109.9985 77.216) (end 108.9025 76.12) (width 0.75) (layer F.Cu) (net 28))
 (segment (start 120.5865 77.216) (end 109.9985 77.216) (width 0.75) (layer F.Cu) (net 28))
 (segment (start 121.9525 75.85) (end 120.5865 77.216) (width 0.75) (layer F.Cu) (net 28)))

